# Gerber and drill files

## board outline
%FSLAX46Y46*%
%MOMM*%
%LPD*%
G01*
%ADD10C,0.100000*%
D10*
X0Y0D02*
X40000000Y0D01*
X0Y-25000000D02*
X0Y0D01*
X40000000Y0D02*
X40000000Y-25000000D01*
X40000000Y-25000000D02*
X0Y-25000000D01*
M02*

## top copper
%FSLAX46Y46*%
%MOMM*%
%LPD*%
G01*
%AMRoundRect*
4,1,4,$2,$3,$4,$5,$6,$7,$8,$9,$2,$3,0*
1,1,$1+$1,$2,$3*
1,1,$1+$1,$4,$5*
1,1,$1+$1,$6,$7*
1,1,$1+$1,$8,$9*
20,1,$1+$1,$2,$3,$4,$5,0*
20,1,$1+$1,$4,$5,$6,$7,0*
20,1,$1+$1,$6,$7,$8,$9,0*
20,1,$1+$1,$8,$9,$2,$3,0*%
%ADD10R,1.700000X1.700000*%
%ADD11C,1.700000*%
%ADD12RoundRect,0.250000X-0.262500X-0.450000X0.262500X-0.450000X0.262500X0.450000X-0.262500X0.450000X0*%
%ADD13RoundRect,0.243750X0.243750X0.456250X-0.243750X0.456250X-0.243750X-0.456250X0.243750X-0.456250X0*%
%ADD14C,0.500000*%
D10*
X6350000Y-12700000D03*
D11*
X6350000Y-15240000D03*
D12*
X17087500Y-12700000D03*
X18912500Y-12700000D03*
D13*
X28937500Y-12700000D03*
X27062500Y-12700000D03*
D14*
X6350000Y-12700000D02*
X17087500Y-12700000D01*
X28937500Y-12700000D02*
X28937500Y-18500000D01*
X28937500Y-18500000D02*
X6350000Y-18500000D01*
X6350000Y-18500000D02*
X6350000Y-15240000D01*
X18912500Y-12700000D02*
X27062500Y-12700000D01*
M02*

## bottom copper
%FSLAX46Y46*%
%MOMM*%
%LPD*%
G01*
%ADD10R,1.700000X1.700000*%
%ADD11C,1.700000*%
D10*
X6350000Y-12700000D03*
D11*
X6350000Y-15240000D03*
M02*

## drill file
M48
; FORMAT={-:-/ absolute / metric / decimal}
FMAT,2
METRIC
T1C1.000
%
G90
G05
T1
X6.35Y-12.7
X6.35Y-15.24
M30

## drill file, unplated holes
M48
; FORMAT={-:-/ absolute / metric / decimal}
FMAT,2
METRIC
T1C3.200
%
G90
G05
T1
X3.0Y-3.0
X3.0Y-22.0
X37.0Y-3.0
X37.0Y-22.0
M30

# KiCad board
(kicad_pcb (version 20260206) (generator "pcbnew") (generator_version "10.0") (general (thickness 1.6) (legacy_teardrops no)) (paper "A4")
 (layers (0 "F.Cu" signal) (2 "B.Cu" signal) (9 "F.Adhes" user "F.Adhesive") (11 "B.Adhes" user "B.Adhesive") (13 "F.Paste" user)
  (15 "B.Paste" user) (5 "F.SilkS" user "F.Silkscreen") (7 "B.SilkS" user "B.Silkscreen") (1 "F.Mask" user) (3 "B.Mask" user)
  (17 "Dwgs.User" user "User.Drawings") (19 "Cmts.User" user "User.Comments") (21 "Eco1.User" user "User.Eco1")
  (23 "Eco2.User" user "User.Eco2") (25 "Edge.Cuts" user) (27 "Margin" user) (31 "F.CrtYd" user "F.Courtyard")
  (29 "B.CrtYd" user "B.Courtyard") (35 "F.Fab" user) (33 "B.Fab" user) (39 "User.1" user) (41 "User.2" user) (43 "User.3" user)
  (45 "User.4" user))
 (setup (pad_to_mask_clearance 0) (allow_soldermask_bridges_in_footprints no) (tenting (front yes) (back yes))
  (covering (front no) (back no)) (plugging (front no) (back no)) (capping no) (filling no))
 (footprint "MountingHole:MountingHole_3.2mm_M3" (layer "F.Cu") (at 3 3)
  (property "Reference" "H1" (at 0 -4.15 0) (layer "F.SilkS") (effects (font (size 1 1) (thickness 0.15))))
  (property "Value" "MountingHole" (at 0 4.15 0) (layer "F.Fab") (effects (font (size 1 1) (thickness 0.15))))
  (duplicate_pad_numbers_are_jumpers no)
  (pad "" np_thru_hole circle (at 0 0) (size 3.2 3.2) (drill 3.2) (layers "*.Cu" "*.Mask")))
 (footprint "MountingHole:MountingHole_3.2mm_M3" (layer "F.Cu") (at 3 22)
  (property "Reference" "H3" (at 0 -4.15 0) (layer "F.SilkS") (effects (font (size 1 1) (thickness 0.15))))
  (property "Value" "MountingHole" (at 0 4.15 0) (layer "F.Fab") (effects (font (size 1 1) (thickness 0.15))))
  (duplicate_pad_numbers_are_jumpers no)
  (pad "" np_thru_hole circle (at 0 0) (size 3.2 3.2) (drill 3.2) (layers "*.Cu" "*.Mask")))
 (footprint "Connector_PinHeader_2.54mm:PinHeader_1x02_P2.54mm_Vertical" (layer "F.Cu") (at 6.35 12.7)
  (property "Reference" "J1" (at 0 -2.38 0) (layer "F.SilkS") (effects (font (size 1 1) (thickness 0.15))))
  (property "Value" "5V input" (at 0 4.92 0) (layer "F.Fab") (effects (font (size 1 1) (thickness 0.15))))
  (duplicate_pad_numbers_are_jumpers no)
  (pad "1" thru_hole rect (at 0 0) (size 1.7 1.7) (drill 1) (layers "*.Cu" "*.Mask") (remove_unused_layers no) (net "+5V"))
  (pad "2" thru_hole circle (at 0 2.54) (size 1.7 1.7) (drill 1) (layers "*.Cu" "*.Mask") (remove_unused_layers no) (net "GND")))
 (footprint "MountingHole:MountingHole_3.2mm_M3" (layer "F.Cu") (at 37 3)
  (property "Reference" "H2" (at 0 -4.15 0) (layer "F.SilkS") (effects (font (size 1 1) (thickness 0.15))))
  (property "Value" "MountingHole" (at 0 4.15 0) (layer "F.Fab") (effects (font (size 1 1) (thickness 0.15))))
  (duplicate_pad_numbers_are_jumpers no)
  (pad "" np_thru_hole circle (at 0 0) (size 3.2 3.2) (drill 3.2) (layers "*.Cu" "*.Mask")))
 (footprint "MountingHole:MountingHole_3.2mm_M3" (layer "F.Cu") (at 37 22)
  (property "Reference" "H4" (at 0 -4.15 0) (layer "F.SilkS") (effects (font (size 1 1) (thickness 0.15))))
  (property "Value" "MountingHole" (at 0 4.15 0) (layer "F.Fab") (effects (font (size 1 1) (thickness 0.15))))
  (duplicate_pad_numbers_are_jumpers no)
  (pad "" np_thru_hole circle (at 0 0) (size 3.2 3.2) (drill 3.2) (layers "*.Cu" "*.Mask")))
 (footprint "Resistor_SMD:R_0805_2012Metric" (layer "F.Cu") (at 18 12.7)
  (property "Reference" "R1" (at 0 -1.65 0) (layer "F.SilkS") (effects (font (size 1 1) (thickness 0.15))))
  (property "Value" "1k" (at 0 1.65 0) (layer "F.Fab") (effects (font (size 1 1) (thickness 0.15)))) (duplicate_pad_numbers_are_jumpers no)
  (pad "1" smd roundrect (at -0.9125 0) (size 1.025 1.4) (layers "F.Cu" "F.Mask" "F.Paste") (roundrect_rratio 0.243902) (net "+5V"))
  (pad "2" smd roundrect (at 0.9125 0) (size 1.025 1.4) (layers "F.Cu" "F.Mask" "F.Paste") (roundrect_rratio 0.243902) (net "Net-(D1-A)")))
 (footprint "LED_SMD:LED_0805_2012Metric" (layer "F.Cu") (at 28 12.7 180)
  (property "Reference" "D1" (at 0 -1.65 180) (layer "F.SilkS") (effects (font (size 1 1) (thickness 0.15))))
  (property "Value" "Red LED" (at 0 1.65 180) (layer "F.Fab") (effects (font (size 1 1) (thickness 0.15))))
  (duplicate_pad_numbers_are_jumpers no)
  (pad "1" smd roundrect (at -0.9375 0 180) (size 0.975 1.4) (layers "F.Cu" "F.Mask" "F.Paste") (roundrect_rratio 0.25) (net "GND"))
  (pad "2" smd roundrect (at 0.9375 0 180) (size 0.975 1.4) (layers "F.Cu" "F.Mask" "F.Paste") (roundrect_rratio 0.25) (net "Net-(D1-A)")))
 (gr_line (start 0 0) (end 40 0) (stroke (width 0.1) (type default)) (layer "Edge.Cuts"))
 (gr_line (start 0 25) (end 0 0) (stroke (width 0.1) (type default)) (layer "Edge.Cuts"))
 (gr_line (start 40 0) (end 40 25) (stroke (width 0.1) (type default)) (layer "Edge.Cuts"))
 (gr_line (start 40 25) (end 0 25) (stroke (width 0.1) (type default)) (layer "Edge.Cuts"))
 (segment (start 6.35 12.7) (end 17.0875 12.7) (width 0.5) (layer "F.Cu") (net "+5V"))
 (segment (start 28.9375 12.7) (end 28.9375 18.5) (width 0.5) (layer "F.Cu") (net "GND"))
 (segment (start 28.9375 18.5) (end 6.35 18.5) (width 0.5) (layer "F.Cu") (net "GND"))
 (segment (start 6.35 18.5) (end 6.35 15.24) (width 0.5) (layer "F.Cu") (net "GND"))
 (segment (start 18.9125 12.7) (end 27.0625 12.7) (width 0.5) (layer "F.Cu") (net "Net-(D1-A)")))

